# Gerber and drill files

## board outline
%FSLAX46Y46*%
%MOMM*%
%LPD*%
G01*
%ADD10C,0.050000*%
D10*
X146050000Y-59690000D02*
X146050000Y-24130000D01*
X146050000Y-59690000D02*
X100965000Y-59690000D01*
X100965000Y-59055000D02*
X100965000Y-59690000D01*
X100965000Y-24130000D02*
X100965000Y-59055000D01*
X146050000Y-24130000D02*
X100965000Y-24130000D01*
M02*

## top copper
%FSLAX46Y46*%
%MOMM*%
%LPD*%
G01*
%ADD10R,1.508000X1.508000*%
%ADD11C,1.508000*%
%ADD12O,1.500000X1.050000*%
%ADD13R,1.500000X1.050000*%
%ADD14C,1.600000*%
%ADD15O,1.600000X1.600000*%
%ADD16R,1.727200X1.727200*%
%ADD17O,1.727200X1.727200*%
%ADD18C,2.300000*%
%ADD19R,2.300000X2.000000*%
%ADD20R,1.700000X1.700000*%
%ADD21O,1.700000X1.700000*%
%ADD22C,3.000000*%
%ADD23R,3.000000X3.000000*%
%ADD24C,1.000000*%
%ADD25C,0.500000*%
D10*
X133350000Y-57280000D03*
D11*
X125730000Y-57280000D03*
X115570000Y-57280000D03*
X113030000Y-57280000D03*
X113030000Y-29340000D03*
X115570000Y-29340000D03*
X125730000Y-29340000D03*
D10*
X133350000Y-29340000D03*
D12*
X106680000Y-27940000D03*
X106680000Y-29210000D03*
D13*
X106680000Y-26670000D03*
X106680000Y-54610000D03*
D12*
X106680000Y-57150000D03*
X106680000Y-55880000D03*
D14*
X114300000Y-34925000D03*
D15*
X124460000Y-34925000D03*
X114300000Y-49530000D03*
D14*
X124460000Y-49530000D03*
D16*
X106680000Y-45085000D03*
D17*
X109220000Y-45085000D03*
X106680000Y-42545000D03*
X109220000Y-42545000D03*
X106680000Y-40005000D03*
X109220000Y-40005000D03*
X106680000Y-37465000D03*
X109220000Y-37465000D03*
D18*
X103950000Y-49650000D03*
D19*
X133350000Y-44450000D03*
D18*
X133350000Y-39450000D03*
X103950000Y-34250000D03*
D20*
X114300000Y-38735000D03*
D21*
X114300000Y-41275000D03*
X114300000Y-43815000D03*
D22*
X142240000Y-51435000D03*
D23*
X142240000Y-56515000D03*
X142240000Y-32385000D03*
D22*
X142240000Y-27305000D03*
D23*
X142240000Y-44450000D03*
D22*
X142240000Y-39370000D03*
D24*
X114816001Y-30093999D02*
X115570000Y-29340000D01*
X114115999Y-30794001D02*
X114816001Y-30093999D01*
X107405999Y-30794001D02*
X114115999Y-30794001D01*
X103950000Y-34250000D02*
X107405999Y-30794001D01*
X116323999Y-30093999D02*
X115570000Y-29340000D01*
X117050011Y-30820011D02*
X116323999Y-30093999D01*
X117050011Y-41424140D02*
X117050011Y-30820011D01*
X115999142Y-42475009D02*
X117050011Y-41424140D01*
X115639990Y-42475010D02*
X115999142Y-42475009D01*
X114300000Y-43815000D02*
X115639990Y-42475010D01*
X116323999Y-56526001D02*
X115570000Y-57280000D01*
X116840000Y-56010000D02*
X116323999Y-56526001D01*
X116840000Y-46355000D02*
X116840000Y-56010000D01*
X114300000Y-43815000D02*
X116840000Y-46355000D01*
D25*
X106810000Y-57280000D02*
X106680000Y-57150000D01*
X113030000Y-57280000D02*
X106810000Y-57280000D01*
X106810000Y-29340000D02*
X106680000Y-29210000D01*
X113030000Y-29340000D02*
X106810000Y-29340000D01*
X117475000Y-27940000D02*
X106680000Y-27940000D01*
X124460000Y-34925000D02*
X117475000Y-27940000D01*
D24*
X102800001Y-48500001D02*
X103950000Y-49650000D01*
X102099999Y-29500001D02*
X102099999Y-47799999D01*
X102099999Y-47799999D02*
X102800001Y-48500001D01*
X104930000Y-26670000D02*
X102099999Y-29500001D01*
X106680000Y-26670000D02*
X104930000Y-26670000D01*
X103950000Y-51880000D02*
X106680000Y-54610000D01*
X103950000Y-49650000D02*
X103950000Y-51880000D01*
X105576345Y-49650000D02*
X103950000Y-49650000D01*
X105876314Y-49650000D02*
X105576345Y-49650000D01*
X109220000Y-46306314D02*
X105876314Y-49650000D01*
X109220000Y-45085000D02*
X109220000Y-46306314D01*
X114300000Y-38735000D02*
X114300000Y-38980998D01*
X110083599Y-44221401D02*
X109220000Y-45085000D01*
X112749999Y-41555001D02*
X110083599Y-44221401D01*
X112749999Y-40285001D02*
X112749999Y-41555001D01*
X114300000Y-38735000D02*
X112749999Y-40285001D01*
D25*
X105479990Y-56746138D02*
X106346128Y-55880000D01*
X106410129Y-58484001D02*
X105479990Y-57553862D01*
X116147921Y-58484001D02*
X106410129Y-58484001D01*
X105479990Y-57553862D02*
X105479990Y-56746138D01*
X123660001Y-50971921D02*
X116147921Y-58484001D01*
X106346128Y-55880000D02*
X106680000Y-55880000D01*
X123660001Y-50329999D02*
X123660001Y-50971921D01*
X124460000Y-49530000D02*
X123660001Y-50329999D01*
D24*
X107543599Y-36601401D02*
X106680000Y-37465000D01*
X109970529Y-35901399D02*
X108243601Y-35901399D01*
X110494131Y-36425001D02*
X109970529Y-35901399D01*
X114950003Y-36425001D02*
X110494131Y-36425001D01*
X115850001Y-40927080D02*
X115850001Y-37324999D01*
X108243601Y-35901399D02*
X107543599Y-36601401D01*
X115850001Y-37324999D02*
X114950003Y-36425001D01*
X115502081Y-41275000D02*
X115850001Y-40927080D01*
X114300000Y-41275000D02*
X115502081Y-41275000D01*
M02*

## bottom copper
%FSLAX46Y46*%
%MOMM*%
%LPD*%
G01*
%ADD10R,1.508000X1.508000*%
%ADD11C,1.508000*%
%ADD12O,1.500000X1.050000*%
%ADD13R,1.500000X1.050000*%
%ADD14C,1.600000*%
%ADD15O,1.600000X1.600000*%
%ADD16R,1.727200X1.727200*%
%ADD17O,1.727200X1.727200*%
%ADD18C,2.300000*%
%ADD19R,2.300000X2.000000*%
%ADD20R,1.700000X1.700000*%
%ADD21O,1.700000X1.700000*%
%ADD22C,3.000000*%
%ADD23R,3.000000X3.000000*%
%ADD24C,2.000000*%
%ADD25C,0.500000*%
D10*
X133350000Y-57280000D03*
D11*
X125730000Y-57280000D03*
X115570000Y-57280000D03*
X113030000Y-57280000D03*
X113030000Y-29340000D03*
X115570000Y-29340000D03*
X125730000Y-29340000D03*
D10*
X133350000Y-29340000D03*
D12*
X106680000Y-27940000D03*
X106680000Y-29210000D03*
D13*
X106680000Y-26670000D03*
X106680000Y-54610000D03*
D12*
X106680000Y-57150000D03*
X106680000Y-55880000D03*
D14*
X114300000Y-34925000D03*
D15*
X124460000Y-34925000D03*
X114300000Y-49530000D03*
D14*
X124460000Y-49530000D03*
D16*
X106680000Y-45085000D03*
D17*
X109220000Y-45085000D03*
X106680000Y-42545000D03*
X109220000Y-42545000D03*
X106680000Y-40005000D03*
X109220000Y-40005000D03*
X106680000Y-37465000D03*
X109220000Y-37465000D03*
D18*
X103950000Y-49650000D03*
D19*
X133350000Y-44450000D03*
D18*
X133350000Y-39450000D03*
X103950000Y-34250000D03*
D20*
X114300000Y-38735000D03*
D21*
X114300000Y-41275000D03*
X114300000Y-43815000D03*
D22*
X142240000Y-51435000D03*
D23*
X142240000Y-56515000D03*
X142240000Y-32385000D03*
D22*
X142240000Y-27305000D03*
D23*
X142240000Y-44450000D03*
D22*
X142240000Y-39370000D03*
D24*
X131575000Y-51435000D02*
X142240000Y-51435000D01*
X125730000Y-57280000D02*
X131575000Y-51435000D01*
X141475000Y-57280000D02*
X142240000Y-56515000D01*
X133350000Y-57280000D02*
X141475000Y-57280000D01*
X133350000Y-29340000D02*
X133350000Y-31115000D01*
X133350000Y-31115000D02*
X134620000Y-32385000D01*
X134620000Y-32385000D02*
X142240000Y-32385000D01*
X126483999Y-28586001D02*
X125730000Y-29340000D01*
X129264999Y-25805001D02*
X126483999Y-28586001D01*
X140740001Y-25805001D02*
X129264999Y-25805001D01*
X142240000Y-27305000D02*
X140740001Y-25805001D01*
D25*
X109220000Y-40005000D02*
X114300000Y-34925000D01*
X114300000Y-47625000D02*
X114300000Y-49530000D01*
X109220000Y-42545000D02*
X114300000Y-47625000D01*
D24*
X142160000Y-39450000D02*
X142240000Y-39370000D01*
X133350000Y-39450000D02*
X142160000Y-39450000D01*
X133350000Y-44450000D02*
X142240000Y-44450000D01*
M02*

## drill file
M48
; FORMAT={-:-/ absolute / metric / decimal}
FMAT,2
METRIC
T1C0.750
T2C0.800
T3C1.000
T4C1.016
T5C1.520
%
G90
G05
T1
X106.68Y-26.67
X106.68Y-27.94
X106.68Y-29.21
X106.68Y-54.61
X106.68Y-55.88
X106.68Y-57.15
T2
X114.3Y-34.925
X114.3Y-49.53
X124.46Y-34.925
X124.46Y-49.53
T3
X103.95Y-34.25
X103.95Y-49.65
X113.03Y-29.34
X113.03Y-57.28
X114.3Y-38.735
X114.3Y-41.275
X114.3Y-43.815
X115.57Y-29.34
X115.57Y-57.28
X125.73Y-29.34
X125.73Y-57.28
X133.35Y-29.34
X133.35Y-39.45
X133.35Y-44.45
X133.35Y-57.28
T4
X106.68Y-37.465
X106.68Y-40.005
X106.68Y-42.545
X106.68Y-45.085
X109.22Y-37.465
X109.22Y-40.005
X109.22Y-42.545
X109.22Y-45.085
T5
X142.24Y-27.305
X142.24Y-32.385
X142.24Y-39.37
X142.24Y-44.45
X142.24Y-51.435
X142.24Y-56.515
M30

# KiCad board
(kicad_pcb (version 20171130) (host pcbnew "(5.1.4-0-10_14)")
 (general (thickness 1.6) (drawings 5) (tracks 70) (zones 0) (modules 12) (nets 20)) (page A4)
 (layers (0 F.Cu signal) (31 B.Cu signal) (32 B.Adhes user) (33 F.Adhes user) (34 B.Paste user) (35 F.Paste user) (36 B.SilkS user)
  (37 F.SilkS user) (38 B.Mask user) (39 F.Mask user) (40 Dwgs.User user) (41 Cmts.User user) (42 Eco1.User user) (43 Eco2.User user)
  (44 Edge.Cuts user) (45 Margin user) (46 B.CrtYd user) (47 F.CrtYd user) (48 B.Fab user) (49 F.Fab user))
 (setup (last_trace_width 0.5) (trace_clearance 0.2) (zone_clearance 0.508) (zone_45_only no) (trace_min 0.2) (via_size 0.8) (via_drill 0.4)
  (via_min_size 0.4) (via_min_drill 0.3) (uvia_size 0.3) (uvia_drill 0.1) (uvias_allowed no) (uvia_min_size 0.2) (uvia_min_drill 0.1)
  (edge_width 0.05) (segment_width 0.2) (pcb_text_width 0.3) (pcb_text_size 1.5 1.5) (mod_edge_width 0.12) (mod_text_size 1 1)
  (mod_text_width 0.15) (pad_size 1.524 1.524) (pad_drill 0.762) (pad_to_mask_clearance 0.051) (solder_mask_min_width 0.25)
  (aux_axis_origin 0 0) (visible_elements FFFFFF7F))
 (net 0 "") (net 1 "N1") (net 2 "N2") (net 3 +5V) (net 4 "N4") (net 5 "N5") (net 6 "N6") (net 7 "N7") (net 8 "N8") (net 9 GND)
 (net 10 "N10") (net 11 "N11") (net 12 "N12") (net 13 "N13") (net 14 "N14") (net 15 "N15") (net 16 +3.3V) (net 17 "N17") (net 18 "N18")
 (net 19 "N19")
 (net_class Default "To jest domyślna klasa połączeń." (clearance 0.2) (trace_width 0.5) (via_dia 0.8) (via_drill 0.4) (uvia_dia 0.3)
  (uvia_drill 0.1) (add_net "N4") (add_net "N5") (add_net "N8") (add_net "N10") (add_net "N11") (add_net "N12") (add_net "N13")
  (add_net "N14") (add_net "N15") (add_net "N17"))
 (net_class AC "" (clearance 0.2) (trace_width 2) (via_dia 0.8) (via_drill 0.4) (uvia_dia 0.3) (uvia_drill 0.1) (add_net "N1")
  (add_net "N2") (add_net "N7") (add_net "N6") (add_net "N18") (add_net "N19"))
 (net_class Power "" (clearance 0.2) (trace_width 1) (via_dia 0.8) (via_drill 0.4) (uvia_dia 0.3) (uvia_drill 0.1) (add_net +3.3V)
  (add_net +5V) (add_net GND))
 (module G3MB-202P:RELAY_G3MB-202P (layer F.Cu) (at 123.19 55.88)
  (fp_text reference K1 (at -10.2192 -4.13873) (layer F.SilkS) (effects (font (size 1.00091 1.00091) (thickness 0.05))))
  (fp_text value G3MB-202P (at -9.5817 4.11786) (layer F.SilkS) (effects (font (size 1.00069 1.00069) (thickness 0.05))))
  (pad 1 thru_hole rect (at 10.16 1.4) (size 1.508 1.508) (drill 1) (layers *.Cu *.Mask) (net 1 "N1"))
  (pad 2 thru_hole circle (at 2.54 1.4) (size 1.508 1.508) (drill 1) (layers *.Cu *.Mask) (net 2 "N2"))
  (pad 3 thru_hole circle (at -7.62 1.4) (size 1.508 1.508) (drill 1) (layers *.Cu *.Mask) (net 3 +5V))
  (pad 4 thru_hole circle (at -10.16 1.4) (size 1.508 1.508) (drill 1) (layers *.Cu *.Mask) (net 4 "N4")))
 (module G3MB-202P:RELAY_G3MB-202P (layer F.Cu) (at 123.19 27.94)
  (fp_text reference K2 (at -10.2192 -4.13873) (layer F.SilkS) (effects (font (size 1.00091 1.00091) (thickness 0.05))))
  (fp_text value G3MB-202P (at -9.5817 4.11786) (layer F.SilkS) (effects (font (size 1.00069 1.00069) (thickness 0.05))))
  (pad 4 thru_hole circle (at -10.16 1.4) (size 1.508 1.508) (drill 1) (layers *.Cu *.Mask) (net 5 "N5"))
  (pad 3 thru_hole circle (at -7.62 1.4) (size 1.508 1.508) (drill 1) (layers *.Cu *.Mask) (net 3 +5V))
  (pad 2 thru_hole circle (at 2.54 1.4) (size 1.508 1.508) (drill 1) (layers *.Cu *.Mask) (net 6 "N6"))
  (pad 1 thru_hole rect (at 10.16 1.4) (size 1.508 1.508) (drill 1) (layers *.Cu *.Mask) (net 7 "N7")))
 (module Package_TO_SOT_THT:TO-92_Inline (layer F.Cu) (at 106.68 26.67 270)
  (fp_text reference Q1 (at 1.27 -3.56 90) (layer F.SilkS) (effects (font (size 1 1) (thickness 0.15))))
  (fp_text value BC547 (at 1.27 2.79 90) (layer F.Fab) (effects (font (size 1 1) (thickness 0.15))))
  (pad 2 thru_hole oval (at 1.27 0 270) (size 1.05 1.5) (drill 0.75) (layers *.Cu *.Mask) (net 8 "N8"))
  (pad 3 thru_hole oval (at 2.54 0 270) (size 1.05 1.5) (drill 0.75) (layers *.Cu *.Mask) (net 5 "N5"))
  (pad 1 thru_hole rect (at 0 0 270) (size 1.05 1.5) (drill 0.75) (layers *.Cu *.Mask) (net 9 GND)))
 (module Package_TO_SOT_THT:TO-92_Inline (layer F.Cu) (at 106.68 54.61 270)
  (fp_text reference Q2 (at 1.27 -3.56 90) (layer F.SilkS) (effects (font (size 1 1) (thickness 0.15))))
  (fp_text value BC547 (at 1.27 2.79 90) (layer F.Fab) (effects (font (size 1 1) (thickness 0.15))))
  (pad 1 thru_hole rect (at 0 0 270) (size 1.05 1.5) (drill 0.75) (layers *.Cu *.Mask) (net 9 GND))
  (pad 3 thru_hole oval (at 2.54 0 270) (size 1.05 1.5) (drill 0.75) (layers *.Cu *.Mask) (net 4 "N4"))
  (pad 2 thru_hole oval (at 1.27 0 270) (size 1.05 1.5) (drill 0.75) (layers *.Cu *.Mask) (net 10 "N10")))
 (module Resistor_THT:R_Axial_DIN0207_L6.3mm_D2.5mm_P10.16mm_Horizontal (layer B.Cu) (at 114.3 34.925)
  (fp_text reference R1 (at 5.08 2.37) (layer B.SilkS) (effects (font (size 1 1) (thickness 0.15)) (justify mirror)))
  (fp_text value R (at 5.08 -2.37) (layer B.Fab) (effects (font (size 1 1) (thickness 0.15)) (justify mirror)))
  (pad 1 thru_hole circle (at 0 0) (size 1.6 1.6) (drill 0.8) (layers *.Cu *.Mask) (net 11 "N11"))
  (pad 2 thru_hole oval (at 10.16 0) (size 1.6 1.6) (drill 0.8) (layers *.Cu *.Mask) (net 8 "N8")))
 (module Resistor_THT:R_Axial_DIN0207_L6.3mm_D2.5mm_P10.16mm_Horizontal (layer B.Cu) (at 124.46 49.53 180)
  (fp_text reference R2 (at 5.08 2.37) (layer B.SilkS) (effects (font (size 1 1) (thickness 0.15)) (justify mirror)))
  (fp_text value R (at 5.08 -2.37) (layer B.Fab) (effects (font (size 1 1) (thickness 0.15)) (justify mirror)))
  (pad 2 thru_hole oval (at 10.16 0 180) (size 1.6 1.6) (drill 0.8) (layers *.Cu *.Mask) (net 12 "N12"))
  (pad 1 thru_hole circle (at 0 0 180) (size 1.6 1.6) (drill 0.8) (layers *.Cu *.Mask) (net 10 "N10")))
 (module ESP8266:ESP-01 (layer B.Cu) (at 106.68 45.085)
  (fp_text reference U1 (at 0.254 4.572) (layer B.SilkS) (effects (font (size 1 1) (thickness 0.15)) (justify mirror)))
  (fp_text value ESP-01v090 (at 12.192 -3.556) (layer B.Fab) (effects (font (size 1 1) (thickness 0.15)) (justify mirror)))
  (pad 1 thru_hole rect (at 0 0) (size 1.7272 1.7272) (drill 1.016) (layers *.Cu *.Mask B.SilkS) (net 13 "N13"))
  (pad 2 thru_hole oval (at 2.54 0) (size 1.7272 1.7272) (drill 1.016) (layers *.Cu *.Mask B.SilkS) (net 9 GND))
  (pad 3 thru_hole oval (at 0 -2.54) (size 1.7272 1.7272) (drill 1.016) (layers *.Cu *.Mask B.SilkS) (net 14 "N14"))
  (pad 4 thru_hole oval (at 2.54 -2.54) (size 1.7272 1.7272) (drill 1.016) (layers *.Cu *.Mask B.SilkS) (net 12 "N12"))
  (pad 5 thru_hole oval (at 0 -5.08) (size 1.7272 1.7272) (drill 1.016) (layers *.Cu *.Mask B.SilkS) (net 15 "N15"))
  (pad 6 thru_hole oval (at 2.54 -5.08) (size 1.7272 1.7272) (drill 1.016) (layers *.Cu *.Mask B.SilkS) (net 11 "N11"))
  (pad 7 thru_hole oval (at 0 -7.62) (size 1.7272 1.7272) (drill 1.016) (layers *.Cu *.Mask B.SilkS) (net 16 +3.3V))
  (pad 8 thru_hole oval (at 2.54 -7.62) (size 1.7272 1.7272) (drill 1.016) (layers *.Cu *.Mask B.SilkS) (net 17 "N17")))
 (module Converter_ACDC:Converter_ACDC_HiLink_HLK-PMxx (layer F.Cu) (at 133.35 44.45 180)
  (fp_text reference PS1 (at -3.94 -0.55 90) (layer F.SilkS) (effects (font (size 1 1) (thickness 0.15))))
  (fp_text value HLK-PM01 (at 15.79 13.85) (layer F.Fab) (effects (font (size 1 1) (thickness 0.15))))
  (pad 3 thru_hole circle (at 29.4 -5.2 180) (size 2.3 2.3) (drill 1) (layers *.Cu *.Mask) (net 9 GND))
  (pad 1 thru_hole rect (at 0 0 180) (size 2.3 2) (drill 1) (layers *.Cu *.Mask) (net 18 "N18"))
  (pad 2 thru_hole circle (at 0 5 180) (size 2.3 2.3) (drill 1) (layers *.Cu *.Mask) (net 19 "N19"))
  (pad 4 thru_hole circle (at 29.4 10.2 180) (size 2.3 2.3) (drill 1) (layers *.Cu *.Mask) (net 3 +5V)))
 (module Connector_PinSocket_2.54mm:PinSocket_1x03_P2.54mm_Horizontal (layer B.Cu) (at 114.3 38.735 180)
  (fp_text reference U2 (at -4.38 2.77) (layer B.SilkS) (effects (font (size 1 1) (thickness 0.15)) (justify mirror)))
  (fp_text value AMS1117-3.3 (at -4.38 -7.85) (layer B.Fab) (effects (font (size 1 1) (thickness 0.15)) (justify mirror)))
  (pad 1 thru_hole rect (at 0 0 180) (size 1.7 1.7) (drill 1) (layers *.Cu *.Mask) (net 9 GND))
  (pad 2 thru_hole oval (at 0 -2.54 180) (size 1.7 1.7) (drill 1) (layers *.Cu *.Mask) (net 16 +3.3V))
  (pad 3 thru_hole oval (at 0 -5.08 180) (size 1.7 1.7) (drill 1) (layers *.Cu *.Mask) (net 3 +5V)))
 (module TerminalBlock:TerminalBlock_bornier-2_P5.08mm (layer F.Cu) (at 142.24 56.515 90)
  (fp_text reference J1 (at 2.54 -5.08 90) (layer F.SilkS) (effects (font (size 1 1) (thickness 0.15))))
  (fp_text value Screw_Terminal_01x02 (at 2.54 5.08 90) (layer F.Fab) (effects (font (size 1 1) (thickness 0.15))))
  (pad 2 thru_hole circle (at 5.08 0 90) (size 3 3) (drill 1.52) (layers *.Cu *.Mask) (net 2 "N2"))
  (pad 1 thru_hole rect (at 0 0 90) (size 3 3) (drill 1.52) (layers *.Cu *.Mask) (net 1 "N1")))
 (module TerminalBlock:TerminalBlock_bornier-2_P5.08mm (layer F.Cu) (at 142.24 32.385 90)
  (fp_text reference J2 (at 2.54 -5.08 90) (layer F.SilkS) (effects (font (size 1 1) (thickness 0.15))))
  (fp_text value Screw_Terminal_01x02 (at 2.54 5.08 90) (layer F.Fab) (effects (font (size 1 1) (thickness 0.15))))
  (pad 1 thru_hole rect (at 0 0 90) (size 3 3) (drill 1.52) (layers *.Cu *.Mask) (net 7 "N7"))
  (pad 2 thru_hole circle (at 5.08 0 90) (size 3 3) (drill 1.52) (layers *.Cu *.Mask) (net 6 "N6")))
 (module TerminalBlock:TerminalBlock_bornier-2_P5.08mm (layer F.Cu) (at 142.24 44.45 90)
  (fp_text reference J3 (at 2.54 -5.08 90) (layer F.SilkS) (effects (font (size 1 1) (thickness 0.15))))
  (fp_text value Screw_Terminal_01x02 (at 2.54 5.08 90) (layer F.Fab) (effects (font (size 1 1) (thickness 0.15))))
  (pad 1 thru_hole rect (at 0 0 90) (size 3 3) (drill 1.52) (layers *.Cu *.Mask) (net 18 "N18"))
  (pad 2 thru_hole circle (at 5.08 0 90) (size 3 3) (drill 1.52) (layers *.Cu *.Mask) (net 19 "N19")))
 (gr_line (start 146.05 59.69) (end 146.05 24.13) (layer Edge.Cuts) (width 0.05))
 (gr_line (start 146.05 59.69) (end 100.965 59.69) (layer Edge.Cuts) (width 0.05))
 (gr_line (start 100.965 59.055) (end 100.965 59.69) (layer Edge.Cuts) (width 0.05))
 (gr_line (start 100.965 24.13) (end 100.965 59.055) (layer Edge.Cuts) (width 0.05))
 (gr_line (start 146.05 24.13) (end 100.965 24.13) (layer Edge.Cuts) (width 0.05))
 (segment (start 131.575 51.435) (end 142.24 51.435) (width 2) (layer B.Cu) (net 2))
 (segment (start 125.73 57.28) (end 131.575 51.435) (width 2) (layer B.Cu) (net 2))
 (segment (start 141.475 57.28) (end 142.24 56.515) (width 2) (layer B.Cu) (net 1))
 (segment (start 133.35 57.28) (end 141.475 57.28) (width 2) (layer B.Cu) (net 1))
 (segment (start 133.35 29.34) (end 133.35 31.115) (width 2) (layer B.Cu) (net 7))
 (segment (start 133.35 31.115) (end 134.62 32.385) (width 2) (layer B.Cu) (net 7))
 (segment (start 134.62 32.385) (end 142.24 32.385) (width 2) (layer B.Cu) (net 7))
 (segment (start 126.483999 28.586001) (end 125.73 29.34) (width 2) (layer B.Cu) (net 6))
 (segment (start 129.264999 25.805001) (end 126.483999 28.586001) (width 2) (layer B.Cu) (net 6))
 (segment (start 140.740001 25.805001) (end 129.264999 25.805001) (width 2) (layer B.Cu) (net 6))
 (segment (start 142.24 27.305) (end 140.740001 25.805001) (width 2) (layer B.Cu) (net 6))
 (segment (start 114.816001 30.093999) (end 115.57 29.34) (width 1) (layer F.Cu) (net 3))
 (segment (start 114.115999 30.794001) (end 114.816001 30.093999) (width 1) (layer F.Cu) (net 3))
 (segment (start 107.405999 30.794001) (end 114.115999 30.794001) (width 1) (layer F.Cu) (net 3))
 (segment (start 103.95 34.25) (end 107.405999 30.794001) (width 1) (layer F.Cu) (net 3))
 (segment (start 116.323999 30.093999) (end 115.57 29.34) (width 1) (layer F.Cu) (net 3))
 (segment (start 117.050011 30.820011) (end 116.323999 30.093999) (width 1) (layer F.Cu) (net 3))
 (segment (start 117.050011 41.42414) (end 117.050011 30.820011) (width 1) (layer F.Cu) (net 3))
 (segment (start 115.999142 42.475009) (end 117.050011 41.42414) (width 1) (layer F.Cu) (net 3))
 (segment (start 115.63999 42.47501) (end 115.999142 42.475009) (width 1) (layer F.Cu) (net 3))
 (segment (start 114.3 43.815) (end 115.63999 42.47501) (width 1) (layer F.Cu) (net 3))
 (segment (start 116.323999 56.526001) (end 115.57 57.28) (width 1) (layer F.Cu) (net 3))
 (segment (start 116.84 56.01) (end 116.323999 56.526001) (width 1) (layer F.Cu) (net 3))
 (segment (start 116.84 46.355) (end 116.84 56.01) (width 1) (layer F.Cu) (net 3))
 (segment (start 114.3 43.815) (end 116.84 46.355) (width 1) (layer F.Cu) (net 3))
 (segment (start 106.81 57.28) (end 106.68 57.15) (width 0.5) (layer F.Cu) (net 4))
 (segment (start 113.03 57.28) (end 106.81 57.28) (width 0.5) (layer F.Cu) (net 4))
 (segment (start 106.81 29.34) (end 106.68 29.21) (width 0.5) (layer F.Cu) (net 5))
 (segment (start 113.03 29.34) (end 106.81 29.34) (width 0.5) (layer F.Cu) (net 5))
 (segment (start 117.475 27.94) (end 106.68 27.94) (width 0.5) (layer F.Cu) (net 8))
 (segment (start 124.46 34.925) (end 117.475 27.94) (width 0.5) (layer F.Cu) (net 8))
 (segment (start 102.800001 48.500001) (end 103.95 49.65) (width 1) (layer F.Cu) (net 9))
 (segment (start 102.099999 29.500001) (end 102.099999 47.799999) (width 1) (layer F.Cu) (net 9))
 (segment (start 102.099999 47.799999) (end 102.800001 48.500001) (width 1) (layer F.Cu) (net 9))
 (segment (start 104.93 26.67) (end 102.099999 29.500001) (width 1) (layer F.Cu) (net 9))
 (segment (start 106.68 26.67) (end 104.93 26.67) (width 1) (layer F.Cu) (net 9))
 (segment (start 103.95 51.88) (end 106.68 54.61) (width 1) (layer F.Cu) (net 9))
 (segment (start 103.95 49.65) (end 103.95 51.88) (width 1) (layer F.Cu) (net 9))
 (segment (start 105.576345 49.65) (end 103.95 49.65) (width 1) (layer F.Cu) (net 9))
 (segment (start 105.876314 49.65) (end 105.576345 49.65) (width 1) (layer F.Cu) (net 9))
 (segment (start 109.22 46.306314) (end 105.876314 49.65) (width 1) (layer F.Cu) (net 9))
 (segment (start 109.22 45.085) (end 109.22 46.306314) (width 1) (layer F.Cu) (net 9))
 (segment (start 114.3 38.735) (end 114.3 38.980998) (width 1) (layer F.Cu) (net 9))
 (segment (start 110.083599 44.221401) (end 109.22 45.085) (width 1) (layer F.Cu) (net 9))
 (segment (start 112.749999 41.555001) (end 110.083599 44.221401) (width 1) (layer F.Cu) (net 9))
 (segment (start 112.749999 40.285001) (end 112.749999 41.555001) (width 1) (layer F.Cu) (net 9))
 (segment (start 114.3 38.735) (end 112.749999 40.285001) (width 1) (layer F.Cu) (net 9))
 (segment (start 105.47999 56.746138) (end 106.346128 55.88) (width 0.5) (layer F.Cu) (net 10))
 (segment (start 106.410129 58.484001) (end 105.47999 57.553862) (width 0.5) (layer F.Cu) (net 10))
 (segment (start 116.147921 58.484001) (end 106.410129 58.484001) (width 0.5) (layer F.Cu) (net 10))
 (segment (start 105.47999 57.553862) (end 105.47999 56.746138) (width 0.5) (layer F.Cu) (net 10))
 (segment (start 123.660001 50.971921) (end 116.147921 58.484001) (width 0.5) (layer F.Cu) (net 10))
 (segment (start 106.346128 55.88) (end 106.68 55.88) (width 0.5) (layer F.Cu) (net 10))
 (segment (start 123.660001 50.329999) (end 123.660001 50.971921) (width 0.5) (layer F.Cu) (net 10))
 (segment (start 124.46 49.53) (end 123.660001 50.329999) (width 0.5) (layer F.Cu) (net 10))
 (segment (start 109.22 40.005) (end 114.3 34.925) (width 0.5) (layer B.Cu) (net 11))
 (segment (start 114.3 47.625) (end 114.3 49.53) (width 0.5) (layer B.Cu) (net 12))
 (segment (start 109.22 42.545) (end 114.3 47.625) (width 0.5) (layer B.Cu) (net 12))
 (segment (start 107.543599 36.601401) (end 106.68 37.465) (width 1) (layer F.Cu) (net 16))
 (segment (start 109.970529 35.901399) (end 108.243601 35.901399) (width 1) (layer F.Cu) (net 16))
 (segment (start 110.494131 36.425001) (end 109.970529 35.901399) (width 1) (layer F.Cu) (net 16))
 (segment (start 114.950003 36.425001) (end 110.494131 36.425001) (width 1) (layer F.Cu) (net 16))
 (segment (start 115.850001 40.92708) (end 115.850001 37.324999) (width 1) (layer F.Cu) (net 16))
 (segment (start 108.243601 35.901399) (end 107.543599 36.601401) (width 1) (layer F.Cu) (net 16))
 (segment (start 115.850001 37.324999) (end 114.950003 36.425001) (width 1) (layer F.Cu) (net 16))
 (segment (start 115.502081 41.275) (end 115.850001 40.92708) (width 1) (layer F.Cu) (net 16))
 (segment (start 114.3 41.275) (end 115.502081 41.275) (width 1) (layer F.Cu) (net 16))
 (segment (start 142.16 39.45) (end 142.24 39.37) (width 2) (layer B.Cu) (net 19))
 (segment (start 133.35 39.45) (end 142.16 39.45) (width 2) (layer B.Cu) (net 19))
 (segment (start 133.35 44.45) (end 142.24 44.45) (width 2) (layer B.Cu) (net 18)))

